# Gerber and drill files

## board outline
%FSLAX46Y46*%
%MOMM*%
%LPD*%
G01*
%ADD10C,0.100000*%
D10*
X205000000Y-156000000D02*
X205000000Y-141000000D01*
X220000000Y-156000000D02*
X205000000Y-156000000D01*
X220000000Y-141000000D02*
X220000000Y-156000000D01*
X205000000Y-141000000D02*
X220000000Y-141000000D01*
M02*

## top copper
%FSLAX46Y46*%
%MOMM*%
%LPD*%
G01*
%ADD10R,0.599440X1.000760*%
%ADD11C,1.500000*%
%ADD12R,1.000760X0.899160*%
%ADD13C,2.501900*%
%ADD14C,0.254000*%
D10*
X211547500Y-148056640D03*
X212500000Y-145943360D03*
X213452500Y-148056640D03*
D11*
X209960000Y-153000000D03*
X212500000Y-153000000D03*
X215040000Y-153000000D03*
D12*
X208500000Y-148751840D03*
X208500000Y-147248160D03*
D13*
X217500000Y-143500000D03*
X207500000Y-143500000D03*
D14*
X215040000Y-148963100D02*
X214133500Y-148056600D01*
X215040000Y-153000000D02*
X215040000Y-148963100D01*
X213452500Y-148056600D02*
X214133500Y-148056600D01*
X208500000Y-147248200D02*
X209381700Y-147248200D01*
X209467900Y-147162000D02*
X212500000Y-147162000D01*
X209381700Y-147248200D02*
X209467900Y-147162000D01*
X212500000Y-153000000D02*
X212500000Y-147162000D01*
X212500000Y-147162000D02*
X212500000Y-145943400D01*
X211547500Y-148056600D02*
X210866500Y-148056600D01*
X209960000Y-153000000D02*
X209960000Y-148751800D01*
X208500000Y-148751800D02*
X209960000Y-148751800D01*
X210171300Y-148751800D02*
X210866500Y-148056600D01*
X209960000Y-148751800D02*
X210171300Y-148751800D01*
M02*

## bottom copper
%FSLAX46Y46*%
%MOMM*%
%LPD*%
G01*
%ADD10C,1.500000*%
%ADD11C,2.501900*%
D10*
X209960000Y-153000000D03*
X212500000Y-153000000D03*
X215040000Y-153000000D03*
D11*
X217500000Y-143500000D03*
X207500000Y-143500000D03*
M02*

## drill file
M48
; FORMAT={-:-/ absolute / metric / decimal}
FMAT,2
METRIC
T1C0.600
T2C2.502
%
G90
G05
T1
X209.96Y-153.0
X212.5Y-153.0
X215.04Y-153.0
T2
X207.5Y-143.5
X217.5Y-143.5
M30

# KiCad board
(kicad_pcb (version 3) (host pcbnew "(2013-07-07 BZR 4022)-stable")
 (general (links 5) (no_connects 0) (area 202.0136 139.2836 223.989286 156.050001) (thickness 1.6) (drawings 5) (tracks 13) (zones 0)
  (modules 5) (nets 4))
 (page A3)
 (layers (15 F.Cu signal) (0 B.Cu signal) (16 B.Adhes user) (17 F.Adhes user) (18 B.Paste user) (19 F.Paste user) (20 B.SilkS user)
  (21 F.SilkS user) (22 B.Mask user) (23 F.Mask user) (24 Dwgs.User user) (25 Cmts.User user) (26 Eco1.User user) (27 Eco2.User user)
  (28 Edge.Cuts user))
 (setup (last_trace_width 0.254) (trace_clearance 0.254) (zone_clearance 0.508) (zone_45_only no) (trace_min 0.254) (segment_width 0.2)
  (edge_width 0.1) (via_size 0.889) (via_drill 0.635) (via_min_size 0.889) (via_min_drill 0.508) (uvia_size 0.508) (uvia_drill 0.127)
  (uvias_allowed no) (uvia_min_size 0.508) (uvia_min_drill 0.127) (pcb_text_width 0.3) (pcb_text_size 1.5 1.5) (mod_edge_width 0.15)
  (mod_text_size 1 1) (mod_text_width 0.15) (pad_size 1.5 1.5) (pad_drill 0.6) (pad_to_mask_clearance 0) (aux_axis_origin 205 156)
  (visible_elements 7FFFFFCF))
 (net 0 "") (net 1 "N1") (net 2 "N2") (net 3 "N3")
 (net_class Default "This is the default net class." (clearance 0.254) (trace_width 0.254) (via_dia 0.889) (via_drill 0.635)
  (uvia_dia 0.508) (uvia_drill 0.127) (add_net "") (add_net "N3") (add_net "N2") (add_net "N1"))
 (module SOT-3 (layer F.Cu) (at 212.5 147)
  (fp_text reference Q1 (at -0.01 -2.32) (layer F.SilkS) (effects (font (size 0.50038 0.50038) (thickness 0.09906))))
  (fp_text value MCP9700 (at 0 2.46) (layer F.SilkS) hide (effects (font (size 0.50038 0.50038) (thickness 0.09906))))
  (pad 1 smd rect (at -0.9525 1.05664) (size 0.59944 1.00076) (layers F.Cu F.Paste F.Mask) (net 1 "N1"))
  (pad 3 smd rect (at 0 -1.05664) (size 0.59944 1.00076) (layers F.Cu F.Paste F.Mask) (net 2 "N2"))
  (pad 2 smd rect (at 0.9525 1.05664) (size 0.59944 1.00076) (layers F.Cu F.Paste F.Mask) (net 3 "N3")))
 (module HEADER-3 (layer F.Cu) (at 212.5 153)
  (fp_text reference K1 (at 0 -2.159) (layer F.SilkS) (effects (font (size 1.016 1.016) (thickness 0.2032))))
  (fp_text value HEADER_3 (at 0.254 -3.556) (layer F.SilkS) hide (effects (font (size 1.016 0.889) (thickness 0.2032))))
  (pad 1 thru_hole circle (at -2.54 0) (size 1.5 1.5) (drill 0.6) (layers *.Cu *.Mask F.SilkS) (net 1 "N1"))
  (pad 2 thru_hole circle (at 0 0) (size 1.5 1.5) (drill 0.6) (layers *.Cu *.Mask F.SilkS) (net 2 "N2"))
  (pad 3 thru_hole circle (at 2.54 0) (size 1.5 1.5) (drill 0.6) (layers *.Cu *.Mask F.SilkS) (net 3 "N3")))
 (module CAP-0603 (layer F.Cu) (at 208.5 148 270)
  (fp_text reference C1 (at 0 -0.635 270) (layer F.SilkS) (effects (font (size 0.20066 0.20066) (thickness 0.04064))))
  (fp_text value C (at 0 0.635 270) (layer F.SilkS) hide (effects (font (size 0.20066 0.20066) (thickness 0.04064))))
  (pad 1 smd rect (at 0.75184 0 270) (size 0.89916 1.00076) (layers F.Cu F.Paste F.Mask) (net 1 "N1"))
  (pad 2 smd rect (at -0.75184 0 270) (size 0.89916 1.00076) (layers F.Cu F.Paste F.Mask) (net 2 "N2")))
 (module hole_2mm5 (layer F.Cu) (at 217.5 143.5)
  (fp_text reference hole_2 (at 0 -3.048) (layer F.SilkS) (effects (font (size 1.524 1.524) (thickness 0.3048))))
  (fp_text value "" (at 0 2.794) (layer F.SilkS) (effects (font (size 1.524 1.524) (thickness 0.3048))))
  (pad 1 thru_hole circle (at 0 0) (size 2.5019 2.5019) (drill 2.5019) (layers *.Cu F.SilkS)))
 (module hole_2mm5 (layer F.Cu) (at 207.5 143.5)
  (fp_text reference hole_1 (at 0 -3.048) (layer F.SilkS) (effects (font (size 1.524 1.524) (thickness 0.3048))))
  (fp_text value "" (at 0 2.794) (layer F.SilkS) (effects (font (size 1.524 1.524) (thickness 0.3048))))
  (pad 1 thru_hole circle (at 0 0) (size 2.5019 2.5019) (drill 2.5019) (layers *.Cu F.SilkS)))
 (gr_line (start 205 156) (end 205 141) (angle 90) (layer Edge.Cuts) (width 0.1))
 (gr_line (start 220 156) (end 205 156) (angle 90) (layer Edge.Cuts) (width 0.1))
 (gr_line (start 220 141) (end 220 156) (angle 90) (layer Edge.Cuts) (width 0.1))
 (gr_line (start 205 141) (end 220 141) (angle 90) (layer Edge.Cuts) (width 0.1))
 (segment (start 215.04 148.9631) (end 214.1335 148.0566) (width 0.254) (layer F.Cu) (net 3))
 (segment (start 215.04 153) (end 215.04 148.9631) (width 0.254) (layer F.Cu) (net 3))
 (segment (start 213.4525 148.0566) (end 214.1335 148.0566) (width 0.254) (layer F.Cu) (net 3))
 (segment (start 208.5 147.2482) (end 209.3817 147.2482) (width 0.254) (layer F.Cu) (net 2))
 (segment (start 209.4679 147.162) (end 212.5 147.162) (width 0.254) (layer F.Cu) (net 2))
 (segment (start 209.3817 147.2482) (end 209.4679 147.162) (width 0.254) (layer F.Cu) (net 2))
 (segment (start 212.5 153) (end 212.5 147.162) (width 0.254) (layer F.Cu) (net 2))
 (segment (start 212.5 147.162) (end 212.5 145.9434) (width 0.254) (layer F.Cu) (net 2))
 (segment (start 211.5475 148.0566) (end 210.8665 148.0566) (width 0.254) (layer F.Cu) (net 1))
 (segment (start 209.96 153) (end 209.96 148.7518) (width 0.254) (layer F.Cu) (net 1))
 (segment (start 208.5 148.7518) (end 209.96 148.7518) (width 0.254) (layer F.Cu) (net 1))
 (segment (start 210.1713 148.7518) (end 210.8665 148.0566) (width 0.254) (layer F.Cu) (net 1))
 (segment (start 209.96 148.7518) (end 210.1713 148.7518) (width 0.254) (layer F.Cu) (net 1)))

